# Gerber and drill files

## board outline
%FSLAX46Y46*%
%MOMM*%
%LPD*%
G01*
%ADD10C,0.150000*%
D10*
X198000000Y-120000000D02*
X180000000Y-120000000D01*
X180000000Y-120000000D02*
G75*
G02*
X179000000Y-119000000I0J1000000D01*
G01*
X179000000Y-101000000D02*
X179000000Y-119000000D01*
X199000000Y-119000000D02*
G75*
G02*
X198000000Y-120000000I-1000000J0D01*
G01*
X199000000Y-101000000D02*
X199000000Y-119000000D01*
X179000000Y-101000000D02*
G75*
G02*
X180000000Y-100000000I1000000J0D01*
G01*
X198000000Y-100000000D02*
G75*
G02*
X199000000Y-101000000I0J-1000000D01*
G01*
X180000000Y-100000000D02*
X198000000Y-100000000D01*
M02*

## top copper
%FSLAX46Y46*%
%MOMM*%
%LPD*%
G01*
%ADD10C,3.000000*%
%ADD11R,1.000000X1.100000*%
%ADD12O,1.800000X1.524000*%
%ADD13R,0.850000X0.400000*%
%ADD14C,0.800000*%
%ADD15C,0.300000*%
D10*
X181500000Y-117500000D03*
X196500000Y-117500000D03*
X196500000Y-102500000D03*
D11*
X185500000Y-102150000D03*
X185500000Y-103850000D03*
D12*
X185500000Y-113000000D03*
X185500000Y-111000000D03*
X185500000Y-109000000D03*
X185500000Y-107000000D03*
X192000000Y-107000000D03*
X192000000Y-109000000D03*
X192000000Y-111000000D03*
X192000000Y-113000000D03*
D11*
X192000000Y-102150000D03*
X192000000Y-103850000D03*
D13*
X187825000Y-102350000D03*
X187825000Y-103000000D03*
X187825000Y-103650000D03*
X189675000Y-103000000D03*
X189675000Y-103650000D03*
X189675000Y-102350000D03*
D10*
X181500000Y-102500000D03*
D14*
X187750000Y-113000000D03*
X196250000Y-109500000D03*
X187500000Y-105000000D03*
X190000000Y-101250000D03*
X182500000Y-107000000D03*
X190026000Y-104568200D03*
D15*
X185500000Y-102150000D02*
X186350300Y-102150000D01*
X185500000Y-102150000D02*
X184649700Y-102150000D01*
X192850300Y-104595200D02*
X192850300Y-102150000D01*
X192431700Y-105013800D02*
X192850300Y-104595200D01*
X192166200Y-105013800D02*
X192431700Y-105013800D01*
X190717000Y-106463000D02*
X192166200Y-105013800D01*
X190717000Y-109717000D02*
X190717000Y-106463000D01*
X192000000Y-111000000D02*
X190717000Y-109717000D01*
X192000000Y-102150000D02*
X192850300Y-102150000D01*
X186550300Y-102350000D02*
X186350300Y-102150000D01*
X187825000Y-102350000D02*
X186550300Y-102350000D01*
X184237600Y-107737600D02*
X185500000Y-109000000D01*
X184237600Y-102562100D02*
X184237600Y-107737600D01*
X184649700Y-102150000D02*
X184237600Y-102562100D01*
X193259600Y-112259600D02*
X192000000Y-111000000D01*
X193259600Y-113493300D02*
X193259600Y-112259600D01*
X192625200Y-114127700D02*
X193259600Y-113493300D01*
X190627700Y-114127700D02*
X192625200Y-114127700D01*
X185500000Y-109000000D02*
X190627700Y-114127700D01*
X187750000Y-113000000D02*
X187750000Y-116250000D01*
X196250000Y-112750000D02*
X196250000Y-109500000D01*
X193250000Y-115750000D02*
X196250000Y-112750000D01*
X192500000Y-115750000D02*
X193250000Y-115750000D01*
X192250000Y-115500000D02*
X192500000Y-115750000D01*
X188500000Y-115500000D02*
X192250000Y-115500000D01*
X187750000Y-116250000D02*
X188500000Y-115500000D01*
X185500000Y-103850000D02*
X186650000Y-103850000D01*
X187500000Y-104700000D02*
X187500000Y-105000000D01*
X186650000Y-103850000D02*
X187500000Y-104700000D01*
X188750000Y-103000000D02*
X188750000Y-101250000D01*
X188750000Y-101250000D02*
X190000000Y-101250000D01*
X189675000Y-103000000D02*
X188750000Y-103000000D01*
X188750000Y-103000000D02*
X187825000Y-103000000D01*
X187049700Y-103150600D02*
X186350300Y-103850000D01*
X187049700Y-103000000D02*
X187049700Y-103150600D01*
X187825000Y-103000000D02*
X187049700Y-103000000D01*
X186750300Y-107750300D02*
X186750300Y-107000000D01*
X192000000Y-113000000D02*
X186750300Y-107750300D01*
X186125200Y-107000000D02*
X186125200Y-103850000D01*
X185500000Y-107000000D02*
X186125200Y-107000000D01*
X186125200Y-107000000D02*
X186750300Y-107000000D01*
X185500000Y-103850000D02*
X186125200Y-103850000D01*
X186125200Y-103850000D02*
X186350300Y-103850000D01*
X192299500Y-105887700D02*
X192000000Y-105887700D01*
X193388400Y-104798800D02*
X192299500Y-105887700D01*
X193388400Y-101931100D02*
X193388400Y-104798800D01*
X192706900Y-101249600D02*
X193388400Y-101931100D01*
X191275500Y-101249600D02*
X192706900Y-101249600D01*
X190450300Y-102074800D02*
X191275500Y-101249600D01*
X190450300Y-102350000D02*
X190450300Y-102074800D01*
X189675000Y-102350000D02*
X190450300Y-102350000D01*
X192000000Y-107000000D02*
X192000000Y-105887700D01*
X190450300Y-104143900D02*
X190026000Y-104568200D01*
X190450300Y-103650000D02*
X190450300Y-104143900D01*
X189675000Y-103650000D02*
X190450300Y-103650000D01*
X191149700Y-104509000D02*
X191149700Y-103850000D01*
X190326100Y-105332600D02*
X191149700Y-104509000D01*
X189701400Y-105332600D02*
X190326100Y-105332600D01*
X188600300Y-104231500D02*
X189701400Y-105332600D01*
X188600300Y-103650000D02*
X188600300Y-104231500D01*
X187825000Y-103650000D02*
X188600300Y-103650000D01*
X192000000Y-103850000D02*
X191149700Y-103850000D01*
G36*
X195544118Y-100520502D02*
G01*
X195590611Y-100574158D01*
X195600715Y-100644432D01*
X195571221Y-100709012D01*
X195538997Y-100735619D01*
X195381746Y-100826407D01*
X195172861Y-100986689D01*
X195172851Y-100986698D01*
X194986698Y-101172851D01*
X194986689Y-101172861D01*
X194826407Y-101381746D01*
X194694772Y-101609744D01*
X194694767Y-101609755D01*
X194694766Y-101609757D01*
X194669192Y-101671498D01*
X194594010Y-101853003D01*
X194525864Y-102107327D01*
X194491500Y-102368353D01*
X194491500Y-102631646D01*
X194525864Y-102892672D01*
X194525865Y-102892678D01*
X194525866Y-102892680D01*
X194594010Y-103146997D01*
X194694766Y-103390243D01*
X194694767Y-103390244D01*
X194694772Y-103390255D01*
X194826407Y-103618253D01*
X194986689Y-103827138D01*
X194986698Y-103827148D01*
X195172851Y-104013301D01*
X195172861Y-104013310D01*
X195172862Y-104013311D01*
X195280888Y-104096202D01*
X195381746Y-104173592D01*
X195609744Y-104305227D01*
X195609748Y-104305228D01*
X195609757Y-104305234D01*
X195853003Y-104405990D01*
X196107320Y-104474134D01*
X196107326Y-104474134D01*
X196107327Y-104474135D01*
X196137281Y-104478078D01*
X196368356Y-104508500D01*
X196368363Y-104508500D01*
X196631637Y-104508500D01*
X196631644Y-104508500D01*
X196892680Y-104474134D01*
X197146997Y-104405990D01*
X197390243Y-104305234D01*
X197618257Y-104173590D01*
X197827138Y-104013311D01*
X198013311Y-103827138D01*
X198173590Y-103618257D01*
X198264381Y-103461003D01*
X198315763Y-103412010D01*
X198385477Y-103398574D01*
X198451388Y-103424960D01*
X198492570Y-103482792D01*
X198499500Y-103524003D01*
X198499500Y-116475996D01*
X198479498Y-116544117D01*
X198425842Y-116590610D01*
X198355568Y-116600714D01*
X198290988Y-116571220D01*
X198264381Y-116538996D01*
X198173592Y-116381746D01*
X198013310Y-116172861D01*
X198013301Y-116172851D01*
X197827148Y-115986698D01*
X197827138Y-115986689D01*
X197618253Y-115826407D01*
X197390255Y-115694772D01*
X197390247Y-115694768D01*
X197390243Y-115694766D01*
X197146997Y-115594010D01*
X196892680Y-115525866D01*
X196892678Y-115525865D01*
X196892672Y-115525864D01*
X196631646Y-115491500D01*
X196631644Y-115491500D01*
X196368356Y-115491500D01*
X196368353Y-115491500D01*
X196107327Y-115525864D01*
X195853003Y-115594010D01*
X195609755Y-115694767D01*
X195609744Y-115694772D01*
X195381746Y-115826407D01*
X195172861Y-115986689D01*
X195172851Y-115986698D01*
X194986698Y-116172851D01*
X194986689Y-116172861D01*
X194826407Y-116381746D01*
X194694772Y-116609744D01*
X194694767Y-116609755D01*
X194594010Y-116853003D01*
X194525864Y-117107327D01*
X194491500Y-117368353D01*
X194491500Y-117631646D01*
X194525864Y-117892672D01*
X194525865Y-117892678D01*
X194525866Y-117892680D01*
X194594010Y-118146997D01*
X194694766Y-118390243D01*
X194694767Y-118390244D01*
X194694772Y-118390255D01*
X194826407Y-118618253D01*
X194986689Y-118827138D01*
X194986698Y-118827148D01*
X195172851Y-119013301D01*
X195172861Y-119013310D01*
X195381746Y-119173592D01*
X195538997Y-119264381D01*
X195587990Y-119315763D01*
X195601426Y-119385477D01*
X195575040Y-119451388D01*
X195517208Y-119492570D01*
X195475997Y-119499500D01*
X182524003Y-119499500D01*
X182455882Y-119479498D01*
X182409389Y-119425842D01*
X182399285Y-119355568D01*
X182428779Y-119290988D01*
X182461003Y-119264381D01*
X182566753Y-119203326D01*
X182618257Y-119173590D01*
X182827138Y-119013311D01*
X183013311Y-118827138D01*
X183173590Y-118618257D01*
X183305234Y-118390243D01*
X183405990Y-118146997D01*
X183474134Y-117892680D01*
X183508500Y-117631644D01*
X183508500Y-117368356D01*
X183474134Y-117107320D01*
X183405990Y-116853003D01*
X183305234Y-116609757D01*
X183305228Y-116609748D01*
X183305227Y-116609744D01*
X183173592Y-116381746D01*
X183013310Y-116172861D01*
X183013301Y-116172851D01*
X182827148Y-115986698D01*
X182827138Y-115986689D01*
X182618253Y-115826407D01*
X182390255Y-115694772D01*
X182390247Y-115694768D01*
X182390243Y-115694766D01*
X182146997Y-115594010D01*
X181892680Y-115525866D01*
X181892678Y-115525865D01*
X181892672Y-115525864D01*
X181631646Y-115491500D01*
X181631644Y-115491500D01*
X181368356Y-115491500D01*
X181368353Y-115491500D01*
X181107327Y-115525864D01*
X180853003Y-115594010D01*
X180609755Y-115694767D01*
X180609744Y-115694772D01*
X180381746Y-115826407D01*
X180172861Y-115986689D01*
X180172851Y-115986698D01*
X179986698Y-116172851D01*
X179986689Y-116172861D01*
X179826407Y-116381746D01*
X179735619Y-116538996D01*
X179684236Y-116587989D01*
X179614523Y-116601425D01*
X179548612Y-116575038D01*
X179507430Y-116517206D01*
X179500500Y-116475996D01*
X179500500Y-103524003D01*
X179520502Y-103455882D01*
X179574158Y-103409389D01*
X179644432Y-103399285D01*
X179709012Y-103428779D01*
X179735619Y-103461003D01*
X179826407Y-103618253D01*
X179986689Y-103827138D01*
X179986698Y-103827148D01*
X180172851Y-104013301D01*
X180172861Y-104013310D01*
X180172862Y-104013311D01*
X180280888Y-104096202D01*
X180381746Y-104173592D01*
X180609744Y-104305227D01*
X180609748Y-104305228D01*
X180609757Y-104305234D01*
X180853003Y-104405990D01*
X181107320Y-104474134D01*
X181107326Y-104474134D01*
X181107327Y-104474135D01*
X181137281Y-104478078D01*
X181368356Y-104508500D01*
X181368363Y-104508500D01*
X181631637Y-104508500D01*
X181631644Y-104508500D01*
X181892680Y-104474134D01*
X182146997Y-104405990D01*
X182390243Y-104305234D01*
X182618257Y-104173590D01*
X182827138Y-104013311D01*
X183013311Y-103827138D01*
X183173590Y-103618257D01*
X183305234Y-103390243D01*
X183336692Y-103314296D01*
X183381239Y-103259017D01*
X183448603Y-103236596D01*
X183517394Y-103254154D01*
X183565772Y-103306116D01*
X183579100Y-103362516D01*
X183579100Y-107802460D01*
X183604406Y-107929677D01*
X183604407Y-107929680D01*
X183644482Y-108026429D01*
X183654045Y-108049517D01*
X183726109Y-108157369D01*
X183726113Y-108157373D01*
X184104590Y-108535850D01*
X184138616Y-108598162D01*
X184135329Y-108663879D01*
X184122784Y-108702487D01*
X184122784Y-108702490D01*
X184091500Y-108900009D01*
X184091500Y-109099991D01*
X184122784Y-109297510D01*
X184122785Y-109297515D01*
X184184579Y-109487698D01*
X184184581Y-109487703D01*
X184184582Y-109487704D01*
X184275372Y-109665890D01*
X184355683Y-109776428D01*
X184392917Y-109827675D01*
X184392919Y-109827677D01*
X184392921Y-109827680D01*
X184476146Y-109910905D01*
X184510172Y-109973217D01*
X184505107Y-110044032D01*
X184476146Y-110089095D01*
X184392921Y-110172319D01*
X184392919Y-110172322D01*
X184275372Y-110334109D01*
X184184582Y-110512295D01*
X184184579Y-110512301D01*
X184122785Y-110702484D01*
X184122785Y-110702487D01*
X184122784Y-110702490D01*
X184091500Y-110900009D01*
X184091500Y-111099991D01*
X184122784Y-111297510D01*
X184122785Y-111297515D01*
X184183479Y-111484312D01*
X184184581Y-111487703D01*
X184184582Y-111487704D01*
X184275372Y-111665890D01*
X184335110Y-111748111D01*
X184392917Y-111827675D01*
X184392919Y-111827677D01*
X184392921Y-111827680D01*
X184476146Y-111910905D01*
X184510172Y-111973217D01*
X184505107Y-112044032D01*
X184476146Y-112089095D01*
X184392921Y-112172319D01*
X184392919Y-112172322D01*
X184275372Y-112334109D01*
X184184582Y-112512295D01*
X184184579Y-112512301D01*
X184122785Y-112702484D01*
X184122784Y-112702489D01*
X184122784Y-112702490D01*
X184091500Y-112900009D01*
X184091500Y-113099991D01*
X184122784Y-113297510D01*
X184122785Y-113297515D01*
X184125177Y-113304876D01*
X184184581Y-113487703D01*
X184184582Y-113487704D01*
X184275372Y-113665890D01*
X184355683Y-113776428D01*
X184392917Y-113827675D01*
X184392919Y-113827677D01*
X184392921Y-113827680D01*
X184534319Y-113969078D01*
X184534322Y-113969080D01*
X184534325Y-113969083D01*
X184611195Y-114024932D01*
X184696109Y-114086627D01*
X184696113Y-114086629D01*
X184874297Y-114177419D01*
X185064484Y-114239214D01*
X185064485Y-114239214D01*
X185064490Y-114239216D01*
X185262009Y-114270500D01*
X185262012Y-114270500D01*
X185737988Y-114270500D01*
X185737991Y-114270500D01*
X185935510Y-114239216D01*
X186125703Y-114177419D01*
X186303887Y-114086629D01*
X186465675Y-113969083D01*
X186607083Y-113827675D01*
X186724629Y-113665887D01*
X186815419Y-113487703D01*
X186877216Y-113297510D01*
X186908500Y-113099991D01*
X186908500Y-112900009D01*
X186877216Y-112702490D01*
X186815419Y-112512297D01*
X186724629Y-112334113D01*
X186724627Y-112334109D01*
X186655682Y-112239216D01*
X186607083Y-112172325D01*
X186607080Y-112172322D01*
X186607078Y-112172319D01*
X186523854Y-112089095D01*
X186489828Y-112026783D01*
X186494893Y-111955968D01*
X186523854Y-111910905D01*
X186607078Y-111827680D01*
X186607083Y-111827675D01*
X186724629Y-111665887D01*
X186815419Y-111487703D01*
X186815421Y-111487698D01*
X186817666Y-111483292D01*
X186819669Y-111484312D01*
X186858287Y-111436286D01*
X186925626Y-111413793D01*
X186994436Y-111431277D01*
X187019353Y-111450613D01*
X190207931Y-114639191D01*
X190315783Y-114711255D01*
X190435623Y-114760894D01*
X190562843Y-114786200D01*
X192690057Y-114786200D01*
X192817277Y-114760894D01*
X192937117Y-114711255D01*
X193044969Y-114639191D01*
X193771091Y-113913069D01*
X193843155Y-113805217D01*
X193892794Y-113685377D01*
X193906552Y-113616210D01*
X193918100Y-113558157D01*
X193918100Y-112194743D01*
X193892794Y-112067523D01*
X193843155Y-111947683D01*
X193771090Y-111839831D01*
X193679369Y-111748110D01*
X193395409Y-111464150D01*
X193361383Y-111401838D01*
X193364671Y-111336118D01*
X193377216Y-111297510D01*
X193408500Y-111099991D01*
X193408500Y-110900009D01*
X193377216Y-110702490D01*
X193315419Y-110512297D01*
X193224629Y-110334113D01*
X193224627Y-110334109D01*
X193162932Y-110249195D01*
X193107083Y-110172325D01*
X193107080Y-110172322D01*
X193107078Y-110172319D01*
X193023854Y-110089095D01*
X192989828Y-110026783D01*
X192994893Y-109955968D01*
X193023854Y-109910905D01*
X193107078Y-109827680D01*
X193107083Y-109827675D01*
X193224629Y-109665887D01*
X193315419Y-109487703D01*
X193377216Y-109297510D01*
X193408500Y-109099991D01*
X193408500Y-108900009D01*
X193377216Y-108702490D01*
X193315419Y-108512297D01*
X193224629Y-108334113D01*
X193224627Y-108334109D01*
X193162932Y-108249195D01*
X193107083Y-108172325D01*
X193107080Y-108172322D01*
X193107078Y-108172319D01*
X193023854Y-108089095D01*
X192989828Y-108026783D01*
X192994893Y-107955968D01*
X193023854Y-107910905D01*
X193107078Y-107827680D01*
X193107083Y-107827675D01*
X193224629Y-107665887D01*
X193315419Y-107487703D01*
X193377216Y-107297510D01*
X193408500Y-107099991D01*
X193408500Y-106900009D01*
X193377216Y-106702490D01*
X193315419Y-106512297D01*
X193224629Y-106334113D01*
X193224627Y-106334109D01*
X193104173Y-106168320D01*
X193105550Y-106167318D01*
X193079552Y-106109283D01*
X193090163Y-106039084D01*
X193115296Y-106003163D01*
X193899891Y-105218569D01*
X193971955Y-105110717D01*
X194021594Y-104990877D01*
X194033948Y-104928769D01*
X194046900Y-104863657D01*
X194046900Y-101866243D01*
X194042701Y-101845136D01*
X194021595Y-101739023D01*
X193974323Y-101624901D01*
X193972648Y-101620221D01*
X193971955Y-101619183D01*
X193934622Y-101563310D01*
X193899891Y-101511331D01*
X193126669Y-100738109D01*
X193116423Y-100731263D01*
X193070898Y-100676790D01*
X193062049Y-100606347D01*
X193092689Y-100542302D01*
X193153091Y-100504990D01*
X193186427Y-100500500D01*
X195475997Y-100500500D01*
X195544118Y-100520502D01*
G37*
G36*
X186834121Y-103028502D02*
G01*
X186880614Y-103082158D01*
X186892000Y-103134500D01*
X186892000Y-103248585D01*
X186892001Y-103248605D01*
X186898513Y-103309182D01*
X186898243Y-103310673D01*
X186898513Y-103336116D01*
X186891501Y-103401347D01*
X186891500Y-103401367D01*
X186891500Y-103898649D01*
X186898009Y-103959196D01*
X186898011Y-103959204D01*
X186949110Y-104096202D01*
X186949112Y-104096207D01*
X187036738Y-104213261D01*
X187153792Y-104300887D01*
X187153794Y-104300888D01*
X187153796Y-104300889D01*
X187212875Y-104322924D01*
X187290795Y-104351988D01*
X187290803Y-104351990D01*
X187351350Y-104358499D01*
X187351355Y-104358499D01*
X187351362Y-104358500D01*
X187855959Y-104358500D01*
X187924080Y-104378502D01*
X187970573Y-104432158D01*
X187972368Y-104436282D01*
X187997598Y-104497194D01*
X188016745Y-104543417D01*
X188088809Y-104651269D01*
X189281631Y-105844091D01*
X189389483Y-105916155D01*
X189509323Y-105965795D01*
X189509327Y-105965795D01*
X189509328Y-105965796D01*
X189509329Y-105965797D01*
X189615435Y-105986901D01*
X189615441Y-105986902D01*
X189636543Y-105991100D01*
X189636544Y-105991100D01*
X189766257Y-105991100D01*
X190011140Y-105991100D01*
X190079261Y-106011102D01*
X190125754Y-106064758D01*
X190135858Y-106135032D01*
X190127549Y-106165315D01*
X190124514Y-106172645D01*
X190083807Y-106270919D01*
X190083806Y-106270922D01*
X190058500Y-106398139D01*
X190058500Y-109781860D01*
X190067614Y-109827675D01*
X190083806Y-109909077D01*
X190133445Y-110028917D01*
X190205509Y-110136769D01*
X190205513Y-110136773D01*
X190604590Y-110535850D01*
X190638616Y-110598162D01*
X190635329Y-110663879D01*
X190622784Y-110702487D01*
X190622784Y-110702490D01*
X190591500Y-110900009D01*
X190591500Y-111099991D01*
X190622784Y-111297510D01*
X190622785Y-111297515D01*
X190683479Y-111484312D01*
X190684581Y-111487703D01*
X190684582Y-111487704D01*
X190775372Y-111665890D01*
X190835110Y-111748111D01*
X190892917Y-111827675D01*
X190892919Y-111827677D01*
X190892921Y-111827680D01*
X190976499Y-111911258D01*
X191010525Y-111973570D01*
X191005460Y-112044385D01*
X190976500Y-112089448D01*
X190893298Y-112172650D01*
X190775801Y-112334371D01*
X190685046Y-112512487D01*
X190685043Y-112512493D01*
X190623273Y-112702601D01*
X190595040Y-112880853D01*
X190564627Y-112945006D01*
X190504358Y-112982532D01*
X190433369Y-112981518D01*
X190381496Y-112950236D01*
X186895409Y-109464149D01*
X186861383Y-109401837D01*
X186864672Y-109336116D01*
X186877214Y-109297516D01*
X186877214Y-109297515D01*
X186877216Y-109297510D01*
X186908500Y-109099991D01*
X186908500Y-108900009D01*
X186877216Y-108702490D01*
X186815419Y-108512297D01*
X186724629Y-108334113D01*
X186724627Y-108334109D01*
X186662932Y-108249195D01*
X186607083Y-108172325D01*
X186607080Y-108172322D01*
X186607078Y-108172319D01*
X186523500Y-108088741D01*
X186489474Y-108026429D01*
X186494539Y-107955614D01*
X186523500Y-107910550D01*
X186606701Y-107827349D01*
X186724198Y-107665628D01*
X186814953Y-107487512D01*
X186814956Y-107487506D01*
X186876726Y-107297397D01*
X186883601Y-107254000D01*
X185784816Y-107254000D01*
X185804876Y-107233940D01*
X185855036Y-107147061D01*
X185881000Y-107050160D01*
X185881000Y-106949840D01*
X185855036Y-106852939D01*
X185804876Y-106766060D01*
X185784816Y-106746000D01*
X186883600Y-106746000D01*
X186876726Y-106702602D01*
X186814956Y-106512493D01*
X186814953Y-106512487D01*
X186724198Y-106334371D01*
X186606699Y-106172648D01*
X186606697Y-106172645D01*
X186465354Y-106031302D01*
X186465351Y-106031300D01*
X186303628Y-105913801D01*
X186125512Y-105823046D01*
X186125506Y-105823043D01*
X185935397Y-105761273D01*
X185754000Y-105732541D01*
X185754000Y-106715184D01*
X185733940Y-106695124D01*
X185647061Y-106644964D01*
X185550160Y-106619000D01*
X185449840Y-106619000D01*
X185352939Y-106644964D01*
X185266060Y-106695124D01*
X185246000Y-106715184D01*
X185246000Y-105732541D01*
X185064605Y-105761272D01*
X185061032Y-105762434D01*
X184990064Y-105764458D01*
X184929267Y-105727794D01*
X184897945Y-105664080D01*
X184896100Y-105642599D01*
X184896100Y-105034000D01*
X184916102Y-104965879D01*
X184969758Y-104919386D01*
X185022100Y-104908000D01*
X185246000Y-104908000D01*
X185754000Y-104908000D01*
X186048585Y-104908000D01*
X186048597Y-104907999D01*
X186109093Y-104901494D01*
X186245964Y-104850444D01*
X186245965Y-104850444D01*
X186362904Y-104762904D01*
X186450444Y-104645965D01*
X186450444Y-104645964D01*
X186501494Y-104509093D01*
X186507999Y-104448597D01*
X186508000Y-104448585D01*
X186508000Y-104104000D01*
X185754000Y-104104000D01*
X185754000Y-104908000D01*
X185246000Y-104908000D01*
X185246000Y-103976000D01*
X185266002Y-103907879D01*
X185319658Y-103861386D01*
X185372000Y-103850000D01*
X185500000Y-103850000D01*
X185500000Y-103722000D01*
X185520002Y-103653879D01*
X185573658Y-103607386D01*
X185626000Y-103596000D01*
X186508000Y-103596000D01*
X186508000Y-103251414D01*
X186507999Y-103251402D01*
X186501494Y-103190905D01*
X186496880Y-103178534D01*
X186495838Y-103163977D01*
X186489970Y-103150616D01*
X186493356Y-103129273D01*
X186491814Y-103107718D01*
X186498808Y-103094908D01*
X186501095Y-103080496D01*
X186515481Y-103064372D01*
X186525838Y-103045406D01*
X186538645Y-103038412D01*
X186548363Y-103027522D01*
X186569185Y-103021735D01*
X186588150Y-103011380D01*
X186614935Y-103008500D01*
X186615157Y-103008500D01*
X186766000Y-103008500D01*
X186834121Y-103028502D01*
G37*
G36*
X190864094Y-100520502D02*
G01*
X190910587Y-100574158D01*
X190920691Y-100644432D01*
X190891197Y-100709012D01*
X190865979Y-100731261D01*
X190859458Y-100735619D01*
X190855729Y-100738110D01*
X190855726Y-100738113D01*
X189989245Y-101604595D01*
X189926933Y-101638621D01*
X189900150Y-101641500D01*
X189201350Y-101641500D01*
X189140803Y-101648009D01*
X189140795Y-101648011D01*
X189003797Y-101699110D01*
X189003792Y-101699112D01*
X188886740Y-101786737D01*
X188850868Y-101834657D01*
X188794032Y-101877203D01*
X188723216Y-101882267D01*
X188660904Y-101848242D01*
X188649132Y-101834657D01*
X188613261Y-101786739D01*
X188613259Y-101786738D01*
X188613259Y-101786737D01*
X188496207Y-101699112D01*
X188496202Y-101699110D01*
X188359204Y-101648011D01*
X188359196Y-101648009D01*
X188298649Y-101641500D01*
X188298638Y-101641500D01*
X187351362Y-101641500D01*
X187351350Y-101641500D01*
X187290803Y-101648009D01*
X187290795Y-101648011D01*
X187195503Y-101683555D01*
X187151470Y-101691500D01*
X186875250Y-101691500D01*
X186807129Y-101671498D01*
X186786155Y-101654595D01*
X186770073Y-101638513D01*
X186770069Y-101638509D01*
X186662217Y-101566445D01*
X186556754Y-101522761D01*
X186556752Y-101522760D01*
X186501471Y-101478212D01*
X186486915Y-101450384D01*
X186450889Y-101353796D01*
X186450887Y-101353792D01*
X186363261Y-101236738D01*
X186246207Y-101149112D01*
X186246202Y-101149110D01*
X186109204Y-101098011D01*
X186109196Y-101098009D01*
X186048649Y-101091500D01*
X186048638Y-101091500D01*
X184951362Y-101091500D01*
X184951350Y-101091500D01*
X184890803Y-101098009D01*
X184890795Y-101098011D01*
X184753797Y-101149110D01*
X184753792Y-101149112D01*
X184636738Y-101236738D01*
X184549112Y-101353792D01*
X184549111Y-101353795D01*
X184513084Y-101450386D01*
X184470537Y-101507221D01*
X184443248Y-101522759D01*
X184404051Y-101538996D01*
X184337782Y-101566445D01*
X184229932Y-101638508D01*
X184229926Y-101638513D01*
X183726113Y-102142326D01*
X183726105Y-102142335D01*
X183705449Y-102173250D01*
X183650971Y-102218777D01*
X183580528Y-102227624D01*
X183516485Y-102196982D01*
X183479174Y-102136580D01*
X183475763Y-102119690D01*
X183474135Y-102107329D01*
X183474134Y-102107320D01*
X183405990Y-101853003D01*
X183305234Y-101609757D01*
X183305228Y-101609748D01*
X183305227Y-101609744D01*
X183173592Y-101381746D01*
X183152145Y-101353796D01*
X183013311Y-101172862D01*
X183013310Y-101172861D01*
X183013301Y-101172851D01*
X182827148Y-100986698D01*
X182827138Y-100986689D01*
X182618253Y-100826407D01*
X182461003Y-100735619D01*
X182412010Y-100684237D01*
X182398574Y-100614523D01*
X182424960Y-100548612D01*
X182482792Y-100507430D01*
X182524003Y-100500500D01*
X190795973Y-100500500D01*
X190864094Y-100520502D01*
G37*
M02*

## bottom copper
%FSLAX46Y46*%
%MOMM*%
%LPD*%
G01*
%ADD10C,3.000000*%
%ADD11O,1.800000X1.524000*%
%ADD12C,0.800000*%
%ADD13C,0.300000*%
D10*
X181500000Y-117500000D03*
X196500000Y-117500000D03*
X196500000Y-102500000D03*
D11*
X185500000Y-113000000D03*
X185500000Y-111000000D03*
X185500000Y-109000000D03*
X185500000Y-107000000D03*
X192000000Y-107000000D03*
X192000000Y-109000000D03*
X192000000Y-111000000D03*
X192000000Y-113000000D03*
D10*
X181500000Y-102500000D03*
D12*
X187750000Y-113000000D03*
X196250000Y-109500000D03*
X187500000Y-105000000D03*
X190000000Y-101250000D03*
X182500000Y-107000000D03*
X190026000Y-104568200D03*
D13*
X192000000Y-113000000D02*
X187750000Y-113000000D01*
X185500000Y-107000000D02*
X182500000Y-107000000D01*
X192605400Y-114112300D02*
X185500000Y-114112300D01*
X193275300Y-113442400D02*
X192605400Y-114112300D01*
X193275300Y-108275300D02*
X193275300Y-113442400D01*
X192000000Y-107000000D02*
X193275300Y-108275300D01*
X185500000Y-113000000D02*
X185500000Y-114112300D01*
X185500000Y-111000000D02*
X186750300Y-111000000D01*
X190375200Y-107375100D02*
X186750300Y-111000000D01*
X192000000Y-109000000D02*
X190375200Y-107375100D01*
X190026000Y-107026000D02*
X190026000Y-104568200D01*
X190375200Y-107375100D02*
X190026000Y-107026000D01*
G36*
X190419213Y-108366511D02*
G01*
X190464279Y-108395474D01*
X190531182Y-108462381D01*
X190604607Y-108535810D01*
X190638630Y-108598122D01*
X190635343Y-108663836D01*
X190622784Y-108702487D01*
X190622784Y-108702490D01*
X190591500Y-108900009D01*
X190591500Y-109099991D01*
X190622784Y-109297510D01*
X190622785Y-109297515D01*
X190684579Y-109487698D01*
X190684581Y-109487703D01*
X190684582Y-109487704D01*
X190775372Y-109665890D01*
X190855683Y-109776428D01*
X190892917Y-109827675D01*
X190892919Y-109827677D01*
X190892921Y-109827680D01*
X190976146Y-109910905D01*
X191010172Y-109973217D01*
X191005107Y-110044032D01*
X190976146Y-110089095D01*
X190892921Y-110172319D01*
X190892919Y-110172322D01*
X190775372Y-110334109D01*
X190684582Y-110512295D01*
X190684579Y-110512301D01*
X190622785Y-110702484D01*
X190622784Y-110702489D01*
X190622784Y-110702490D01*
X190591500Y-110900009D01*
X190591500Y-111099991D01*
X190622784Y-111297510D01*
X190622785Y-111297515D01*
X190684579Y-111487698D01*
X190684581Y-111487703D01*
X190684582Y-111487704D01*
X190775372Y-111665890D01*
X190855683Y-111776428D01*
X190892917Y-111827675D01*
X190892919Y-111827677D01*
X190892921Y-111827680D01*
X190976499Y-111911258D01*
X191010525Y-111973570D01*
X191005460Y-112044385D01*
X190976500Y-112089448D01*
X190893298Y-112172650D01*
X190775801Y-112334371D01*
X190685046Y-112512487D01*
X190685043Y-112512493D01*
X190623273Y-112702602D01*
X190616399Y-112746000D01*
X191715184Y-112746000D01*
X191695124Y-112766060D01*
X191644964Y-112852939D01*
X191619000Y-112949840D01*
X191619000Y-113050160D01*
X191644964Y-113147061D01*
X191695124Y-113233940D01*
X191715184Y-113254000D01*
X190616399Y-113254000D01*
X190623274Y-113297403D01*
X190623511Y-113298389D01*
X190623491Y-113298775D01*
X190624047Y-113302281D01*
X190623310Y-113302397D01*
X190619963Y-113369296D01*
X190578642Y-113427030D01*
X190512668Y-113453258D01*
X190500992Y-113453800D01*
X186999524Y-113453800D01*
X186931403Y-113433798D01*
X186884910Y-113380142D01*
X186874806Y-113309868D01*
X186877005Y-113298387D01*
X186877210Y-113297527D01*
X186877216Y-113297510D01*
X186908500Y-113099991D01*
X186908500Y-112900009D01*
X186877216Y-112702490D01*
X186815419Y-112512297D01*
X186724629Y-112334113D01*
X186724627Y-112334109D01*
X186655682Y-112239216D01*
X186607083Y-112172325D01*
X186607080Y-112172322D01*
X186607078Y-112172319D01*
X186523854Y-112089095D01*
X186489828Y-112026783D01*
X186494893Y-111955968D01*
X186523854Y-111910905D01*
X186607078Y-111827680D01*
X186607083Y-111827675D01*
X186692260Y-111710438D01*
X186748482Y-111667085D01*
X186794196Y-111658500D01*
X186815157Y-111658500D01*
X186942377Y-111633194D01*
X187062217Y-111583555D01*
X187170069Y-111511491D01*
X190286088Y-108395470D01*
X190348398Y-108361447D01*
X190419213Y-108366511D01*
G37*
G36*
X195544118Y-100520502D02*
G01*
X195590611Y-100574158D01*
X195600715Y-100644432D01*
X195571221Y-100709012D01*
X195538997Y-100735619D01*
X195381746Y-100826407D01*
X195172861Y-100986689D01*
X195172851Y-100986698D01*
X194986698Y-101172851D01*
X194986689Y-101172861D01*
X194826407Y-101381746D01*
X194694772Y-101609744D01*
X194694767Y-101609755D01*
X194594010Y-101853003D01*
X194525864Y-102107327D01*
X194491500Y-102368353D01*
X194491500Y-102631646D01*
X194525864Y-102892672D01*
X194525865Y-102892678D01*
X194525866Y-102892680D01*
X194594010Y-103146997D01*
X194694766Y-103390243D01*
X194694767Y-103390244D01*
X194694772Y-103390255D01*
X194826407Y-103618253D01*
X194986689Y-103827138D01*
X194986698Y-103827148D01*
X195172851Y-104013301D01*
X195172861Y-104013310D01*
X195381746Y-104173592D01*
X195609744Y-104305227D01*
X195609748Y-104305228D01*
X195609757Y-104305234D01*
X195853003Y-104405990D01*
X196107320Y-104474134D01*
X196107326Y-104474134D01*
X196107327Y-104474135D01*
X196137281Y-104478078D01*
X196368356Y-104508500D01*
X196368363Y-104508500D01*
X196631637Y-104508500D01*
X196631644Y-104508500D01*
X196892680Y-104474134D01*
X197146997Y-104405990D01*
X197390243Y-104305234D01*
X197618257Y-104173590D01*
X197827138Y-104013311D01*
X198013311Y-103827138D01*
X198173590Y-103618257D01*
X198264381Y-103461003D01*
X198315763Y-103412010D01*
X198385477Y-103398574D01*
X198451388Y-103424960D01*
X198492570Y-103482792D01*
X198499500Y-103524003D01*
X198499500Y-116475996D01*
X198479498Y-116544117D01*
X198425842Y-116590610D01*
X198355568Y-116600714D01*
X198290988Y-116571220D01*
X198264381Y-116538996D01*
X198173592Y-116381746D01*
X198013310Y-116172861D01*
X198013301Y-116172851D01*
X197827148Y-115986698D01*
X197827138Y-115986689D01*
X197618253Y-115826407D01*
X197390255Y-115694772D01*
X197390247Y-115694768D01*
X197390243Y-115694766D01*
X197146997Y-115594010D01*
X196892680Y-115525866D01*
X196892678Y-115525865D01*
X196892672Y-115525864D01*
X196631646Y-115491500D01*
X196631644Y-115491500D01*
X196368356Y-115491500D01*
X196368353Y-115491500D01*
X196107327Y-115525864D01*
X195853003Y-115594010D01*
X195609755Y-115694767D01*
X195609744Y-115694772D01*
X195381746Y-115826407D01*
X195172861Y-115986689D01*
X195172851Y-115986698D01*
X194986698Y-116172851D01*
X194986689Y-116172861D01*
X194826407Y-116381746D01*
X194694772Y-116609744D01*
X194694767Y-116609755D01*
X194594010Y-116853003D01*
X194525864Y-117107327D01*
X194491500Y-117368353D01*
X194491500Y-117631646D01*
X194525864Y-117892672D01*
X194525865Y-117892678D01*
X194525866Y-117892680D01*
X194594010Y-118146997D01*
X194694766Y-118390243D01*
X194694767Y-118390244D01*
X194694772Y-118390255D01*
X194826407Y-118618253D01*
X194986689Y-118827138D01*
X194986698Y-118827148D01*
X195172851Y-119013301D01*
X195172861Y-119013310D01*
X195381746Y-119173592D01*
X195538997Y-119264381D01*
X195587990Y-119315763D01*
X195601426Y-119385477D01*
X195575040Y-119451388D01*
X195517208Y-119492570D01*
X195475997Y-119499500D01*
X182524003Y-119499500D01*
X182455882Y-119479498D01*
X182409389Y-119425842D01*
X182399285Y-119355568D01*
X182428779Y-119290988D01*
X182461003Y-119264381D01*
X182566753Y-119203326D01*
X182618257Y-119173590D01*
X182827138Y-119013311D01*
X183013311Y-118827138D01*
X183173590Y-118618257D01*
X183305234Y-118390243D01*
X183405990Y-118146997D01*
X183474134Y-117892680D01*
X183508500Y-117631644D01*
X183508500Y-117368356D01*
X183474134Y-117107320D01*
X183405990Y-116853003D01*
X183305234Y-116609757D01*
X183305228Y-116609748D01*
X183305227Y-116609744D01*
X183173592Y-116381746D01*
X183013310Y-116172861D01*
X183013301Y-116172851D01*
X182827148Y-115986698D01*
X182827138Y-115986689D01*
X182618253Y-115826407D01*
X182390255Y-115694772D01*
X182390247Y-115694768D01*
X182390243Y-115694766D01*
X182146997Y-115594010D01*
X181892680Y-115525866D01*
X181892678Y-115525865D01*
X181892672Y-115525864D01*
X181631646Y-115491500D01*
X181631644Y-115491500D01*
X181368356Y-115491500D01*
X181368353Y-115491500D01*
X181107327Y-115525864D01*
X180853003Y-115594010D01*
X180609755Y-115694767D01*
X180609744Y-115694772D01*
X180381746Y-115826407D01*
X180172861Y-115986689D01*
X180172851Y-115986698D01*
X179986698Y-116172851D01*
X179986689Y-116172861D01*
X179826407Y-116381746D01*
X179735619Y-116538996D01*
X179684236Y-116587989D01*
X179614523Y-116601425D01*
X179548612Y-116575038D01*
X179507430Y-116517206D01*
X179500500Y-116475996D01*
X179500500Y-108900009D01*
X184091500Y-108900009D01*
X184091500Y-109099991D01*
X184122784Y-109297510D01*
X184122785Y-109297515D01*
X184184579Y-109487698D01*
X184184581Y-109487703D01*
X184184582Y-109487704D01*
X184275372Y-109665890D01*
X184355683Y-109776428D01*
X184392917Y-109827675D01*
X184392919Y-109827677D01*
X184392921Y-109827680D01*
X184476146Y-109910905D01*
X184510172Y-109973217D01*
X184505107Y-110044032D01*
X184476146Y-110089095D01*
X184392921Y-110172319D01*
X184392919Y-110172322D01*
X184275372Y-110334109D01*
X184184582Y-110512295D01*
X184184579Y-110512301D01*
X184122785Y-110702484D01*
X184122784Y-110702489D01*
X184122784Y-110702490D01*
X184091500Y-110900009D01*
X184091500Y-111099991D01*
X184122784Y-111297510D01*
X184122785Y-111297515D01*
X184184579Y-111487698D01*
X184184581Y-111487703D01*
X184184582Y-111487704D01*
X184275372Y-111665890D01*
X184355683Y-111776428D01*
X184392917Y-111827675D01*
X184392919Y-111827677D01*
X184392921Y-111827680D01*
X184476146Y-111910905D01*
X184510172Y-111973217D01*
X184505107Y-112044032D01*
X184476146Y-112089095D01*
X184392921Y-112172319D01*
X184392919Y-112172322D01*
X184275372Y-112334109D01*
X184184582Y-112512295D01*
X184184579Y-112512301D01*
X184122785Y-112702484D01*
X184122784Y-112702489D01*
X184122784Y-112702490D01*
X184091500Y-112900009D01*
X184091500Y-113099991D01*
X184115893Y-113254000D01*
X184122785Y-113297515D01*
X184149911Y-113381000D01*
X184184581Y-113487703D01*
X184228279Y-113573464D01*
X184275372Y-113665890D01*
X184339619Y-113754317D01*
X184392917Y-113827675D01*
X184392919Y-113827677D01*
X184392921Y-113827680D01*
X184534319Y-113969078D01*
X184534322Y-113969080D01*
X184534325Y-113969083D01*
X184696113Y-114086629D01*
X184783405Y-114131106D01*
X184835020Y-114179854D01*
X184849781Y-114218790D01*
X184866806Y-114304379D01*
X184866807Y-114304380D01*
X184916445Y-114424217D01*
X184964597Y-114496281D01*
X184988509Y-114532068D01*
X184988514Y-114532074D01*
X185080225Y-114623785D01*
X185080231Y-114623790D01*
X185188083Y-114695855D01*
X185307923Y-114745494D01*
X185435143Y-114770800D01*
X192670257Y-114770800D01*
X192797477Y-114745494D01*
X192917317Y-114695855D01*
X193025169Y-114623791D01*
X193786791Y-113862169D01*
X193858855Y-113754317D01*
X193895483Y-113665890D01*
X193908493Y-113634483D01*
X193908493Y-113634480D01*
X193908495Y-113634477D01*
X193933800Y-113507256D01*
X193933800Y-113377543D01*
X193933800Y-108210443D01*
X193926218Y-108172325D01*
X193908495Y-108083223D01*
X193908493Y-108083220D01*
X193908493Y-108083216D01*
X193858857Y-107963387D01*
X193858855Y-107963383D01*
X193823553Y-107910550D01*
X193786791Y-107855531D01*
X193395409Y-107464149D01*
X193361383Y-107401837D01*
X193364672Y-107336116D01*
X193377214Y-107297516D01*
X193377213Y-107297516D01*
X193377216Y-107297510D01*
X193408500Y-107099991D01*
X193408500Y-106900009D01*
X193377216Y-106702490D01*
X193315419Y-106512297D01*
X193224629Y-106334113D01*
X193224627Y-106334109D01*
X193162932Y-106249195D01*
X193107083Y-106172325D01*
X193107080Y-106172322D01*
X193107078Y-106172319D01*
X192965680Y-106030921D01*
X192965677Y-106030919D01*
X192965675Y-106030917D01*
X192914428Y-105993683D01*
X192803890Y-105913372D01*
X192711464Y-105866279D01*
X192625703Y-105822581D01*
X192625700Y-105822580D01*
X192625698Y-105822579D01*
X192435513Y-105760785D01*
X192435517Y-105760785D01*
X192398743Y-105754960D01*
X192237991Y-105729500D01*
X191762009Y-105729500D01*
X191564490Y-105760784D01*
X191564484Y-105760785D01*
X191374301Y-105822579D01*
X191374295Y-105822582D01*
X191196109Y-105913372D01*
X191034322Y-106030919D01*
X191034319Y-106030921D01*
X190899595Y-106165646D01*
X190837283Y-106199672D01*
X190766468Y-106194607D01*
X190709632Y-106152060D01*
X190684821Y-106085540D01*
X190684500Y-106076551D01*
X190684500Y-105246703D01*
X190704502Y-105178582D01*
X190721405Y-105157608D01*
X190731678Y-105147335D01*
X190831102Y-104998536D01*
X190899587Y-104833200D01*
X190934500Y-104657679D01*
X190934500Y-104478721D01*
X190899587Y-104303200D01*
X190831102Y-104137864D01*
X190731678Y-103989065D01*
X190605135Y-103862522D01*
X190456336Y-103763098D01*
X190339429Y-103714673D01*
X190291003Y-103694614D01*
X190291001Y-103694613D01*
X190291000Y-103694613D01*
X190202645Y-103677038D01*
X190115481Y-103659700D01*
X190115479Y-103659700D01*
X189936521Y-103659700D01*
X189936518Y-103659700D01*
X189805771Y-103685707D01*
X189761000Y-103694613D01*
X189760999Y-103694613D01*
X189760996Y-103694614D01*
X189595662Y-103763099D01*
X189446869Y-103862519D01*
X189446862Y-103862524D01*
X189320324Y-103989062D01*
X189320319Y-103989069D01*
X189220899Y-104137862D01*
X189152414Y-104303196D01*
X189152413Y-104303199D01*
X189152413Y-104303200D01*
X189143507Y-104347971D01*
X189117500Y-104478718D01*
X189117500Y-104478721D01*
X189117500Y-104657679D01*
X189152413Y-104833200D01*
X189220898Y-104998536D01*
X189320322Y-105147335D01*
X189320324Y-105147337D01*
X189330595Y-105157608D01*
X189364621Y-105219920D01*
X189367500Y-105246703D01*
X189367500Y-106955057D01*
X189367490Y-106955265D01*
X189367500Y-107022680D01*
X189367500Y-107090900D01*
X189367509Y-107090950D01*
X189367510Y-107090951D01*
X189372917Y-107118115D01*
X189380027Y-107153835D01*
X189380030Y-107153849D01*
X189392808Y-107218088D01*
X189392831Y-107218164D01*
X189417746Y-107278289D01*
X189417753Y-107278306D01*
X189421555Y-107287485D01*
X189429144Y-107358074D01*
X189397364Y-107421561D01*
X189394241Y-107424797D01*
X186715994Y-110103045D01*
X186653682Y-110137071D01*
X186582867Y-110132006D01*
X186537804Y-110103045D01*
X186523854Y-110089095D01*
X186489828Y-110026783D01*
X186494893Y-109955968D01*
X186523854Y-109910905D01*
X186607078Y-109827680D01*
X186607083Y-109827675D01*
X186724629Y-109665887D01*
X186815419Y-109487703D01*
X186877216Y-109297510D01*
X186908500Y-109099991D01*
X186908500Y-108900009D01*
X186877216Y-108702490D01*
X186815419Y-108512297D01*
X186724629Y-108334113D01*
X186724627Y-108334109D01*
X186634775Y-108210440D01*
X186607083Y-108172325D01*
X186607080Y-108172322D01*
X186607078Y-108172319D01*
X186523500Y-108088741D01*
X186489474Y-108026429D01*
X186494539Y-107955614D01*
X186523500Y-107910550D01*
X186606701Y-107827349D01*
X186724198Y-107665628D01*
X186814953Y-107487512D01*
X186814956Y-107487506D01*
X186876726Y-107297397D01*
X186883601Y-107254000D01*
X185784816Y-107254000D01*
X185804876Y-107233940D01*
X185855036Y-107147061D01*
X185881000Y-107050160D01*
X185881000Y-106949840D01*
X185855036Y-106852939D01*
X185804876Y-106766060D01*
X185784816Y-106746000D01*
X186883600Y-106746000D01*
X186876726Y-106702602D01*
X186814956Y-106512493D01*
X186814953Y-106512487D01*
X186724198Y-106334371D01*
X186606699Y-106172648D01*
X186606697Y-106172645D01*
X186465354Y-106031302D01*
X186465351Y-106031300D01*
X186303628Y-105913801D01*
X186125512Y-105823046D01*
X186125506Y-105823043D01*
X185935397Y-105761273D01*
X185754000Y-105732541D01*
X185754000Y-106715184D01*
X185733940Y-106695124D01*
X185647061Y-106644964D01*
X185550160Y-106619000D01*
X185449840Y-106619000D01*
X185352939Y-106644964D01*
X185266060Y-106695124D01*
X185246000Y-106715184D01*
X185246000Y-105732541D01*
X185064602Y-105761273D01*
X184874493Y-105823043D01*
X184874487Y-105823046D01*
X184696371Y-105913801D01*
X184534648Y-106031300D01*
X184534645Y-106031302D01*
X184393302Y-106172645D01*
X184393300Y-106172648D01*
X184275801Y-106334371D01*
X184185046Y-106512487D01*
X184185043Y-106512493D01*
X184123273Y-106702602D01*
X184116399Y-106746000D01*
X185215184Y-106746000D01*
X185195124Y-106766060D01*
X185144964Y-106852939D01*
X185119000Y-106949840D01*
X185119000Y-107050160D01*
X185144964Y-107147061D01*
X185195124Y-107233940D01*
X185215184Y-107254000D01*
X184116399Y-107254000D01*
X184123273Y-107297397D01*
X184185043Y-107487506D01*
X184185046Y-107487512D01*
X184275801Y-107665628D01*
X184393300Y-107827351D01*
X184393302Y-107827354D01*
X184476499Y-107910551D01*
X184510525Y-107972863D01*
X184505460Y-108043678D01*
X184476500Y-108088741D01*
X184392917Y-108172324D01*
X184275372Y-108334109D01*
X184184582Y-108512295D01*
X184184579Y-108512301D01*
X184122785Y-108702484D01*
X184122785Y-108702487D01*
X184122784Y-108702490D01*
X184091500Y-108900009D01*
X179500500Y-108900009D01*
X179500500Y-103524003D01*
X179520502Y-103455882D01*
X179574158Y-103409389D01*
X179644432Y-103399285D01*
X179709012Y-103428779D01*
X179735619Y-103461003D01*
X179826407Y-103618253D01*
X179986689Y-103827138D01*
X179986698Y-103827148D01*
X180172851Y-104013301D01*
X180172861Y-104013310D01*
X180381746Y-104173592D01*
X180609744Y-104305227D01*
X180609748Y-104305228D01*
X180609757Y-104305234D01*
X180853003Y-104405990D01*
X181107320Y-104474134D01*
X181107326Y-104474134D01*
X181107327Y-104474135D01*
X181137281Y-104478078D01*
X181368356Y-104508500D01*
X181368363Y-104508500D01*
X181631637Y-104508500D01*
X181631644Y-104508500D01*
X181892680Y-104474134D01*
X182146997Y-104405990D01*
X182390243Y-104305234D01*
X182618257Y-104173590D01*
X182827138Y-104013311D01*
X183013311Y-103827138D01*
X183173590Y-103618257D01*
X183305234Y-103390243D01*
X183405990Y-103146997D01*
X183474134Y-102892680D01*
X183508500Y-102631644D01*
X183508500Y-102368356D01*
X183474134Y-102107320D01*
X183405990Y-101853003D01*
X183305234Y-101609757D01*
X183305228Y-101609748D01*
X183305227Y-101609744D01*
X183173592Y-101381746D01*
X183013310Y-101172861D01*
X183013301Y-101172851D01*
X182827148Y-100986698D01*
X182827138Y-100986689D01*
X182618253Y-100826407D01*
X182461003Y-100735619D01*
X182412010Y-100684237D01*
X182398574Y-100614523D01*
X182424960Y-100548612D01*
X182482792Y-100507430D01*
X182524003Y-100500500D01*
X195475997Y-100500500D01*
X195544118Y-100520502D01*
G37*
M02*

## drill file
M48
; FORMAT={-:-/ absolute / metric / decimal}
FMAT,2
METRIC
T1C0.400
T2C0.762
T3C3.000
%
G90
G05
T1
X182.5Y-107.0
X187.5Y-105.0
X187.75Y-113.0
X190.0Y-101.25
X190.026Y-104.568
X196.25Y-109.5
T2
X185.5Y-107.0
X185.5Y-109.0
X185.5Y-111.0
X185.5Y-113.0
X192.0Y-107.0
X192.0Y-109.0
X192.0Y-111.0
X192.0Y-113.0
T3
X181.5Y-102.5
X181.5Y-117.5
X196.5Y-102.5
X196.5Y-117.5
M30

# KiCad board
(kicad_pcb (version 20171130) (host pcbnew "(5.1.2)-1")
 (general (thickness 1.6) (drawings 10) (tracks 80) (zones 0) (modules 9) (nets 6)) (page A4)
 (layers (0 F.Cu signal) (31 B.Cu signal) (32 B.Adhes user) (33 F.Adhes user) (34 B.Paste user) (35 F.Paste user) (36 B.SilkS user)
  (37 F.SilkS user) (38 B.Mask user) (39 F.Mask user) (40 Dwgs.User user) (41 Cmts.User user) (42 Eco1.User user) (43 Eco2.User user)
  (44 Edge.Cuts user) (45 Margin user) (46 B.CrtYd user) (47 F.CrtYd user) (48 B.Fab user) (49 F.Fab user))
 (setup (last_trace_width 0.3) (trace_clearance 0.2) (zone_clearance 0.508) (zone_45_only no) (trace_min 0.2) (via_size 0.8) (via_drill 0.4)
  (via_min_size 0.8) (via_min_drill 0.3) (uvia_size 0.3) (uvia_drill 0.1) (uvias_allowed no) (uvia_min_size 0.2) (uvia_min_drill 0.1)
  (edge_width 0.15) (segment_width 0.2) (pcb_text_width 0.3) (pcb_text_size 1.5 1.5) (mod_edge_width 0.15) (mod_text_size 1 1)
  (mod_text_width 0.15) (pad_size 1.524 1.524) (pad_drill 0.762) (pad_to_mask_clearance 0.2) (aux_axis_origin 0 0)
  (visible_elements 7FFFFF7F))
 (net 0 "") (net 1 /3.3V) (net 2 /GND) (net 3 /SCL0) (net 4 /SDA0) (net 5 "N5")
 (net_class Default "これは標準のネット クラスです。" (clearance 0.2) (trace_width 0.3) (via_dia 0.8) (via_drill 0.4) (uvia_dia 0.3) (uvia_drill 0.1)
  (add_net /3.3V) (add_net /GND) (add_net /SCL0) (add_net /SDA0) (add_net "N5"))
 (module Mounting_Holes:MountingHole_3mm (layer F.Cu) (at 181.5 117.5)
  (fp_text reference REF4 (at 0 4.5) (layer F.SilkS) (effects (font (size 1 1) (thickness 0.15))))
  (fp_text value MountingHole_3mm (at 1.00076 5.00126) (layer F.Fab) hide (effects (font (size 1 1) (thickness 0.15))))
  (pad 1 thru_hole circle (at 0 0) (size 3 3) (drill 3) (layers)))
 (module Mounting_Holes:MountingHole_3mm (layer F.Cu) (at 196.5 117.5)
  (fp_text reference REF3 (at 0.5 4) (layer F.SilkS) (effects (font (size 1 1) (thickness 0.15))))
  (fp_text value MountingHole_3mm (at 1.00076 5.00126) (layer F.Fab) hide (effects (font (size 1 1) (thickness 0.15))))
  (pad 1 thru_hole circle (at 0 0) (size 3 3) (drill 3) (layers)))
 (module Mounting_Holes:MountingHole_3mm (layer F.Cu) (at 196.5 102.5)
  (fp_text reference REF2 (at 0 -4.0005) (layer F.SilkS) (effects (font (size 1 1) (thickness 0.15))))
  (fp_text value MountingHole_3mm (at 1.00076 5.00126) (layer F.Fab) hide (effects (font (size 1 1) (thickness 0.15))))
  (pad 1 thru_hole circle (at 0 0) (size 3 3) (drill 3) (layers)))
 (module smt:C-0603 (layer F.Cu) (at 185.5 103 270)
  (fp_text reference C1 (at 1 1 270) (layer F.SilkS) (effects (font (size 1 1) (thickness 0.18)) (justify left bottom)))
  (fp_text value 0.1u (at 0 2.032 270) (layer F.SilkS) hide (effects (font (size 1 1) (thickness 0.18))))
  (pad 1 smd rect (at -0.85 0 270) (size 1.1 1) (layers F.Cu F.Paste F.Mask) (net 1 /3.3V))
  (pad 2 smd rect (at 0.85 0 270) (size 1.1 1) (layers F.Cu F.Paste F.Mask) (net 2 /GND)))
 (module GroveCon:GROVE (layer F.Cu) (at 185.5 113 90)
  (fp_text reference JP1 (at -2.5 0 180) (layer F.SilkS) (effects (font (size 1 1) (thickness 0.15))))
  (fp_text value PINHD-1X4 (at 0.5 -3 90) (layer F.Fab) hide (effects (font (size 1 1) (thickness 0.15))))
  (pad 1 thru_hole oval (at 0 0 90) (size 1.524 1.8) (drill 0.762) (layers *.Cu *.Paste *.Mask F.SilkS) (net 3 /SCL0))
  (pad 2 thru_hole oval (at 2 0 90) (size 1.524 1.8) (drill 0.762) (layers *.Cu *.Paste *.Mask F.SilkS) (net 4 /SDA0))
  (pad 3 thru_hole oval (at 4 0 90) (size 1.524 1.8) (drill 0.762) (layers *.Cu *.Paste *.Mask F.SilkS) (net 1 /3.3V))
  (pad 4 thru_hole oval (at 6 0 90) (size 1.524 1.8) (drill 0.762) (layers *.Cu *.Paste *.Mask F.SilkS) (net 2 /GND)))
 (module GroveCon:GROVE (layer F.Cu) (at 192 107 270)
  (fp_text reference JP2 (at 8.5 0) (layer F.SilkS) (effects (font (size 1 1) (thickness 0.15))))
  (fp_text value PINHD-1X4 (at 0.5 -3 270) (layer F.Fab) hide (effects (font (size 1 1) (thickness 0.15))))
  (pad 1 thru_hole oval (at 0 0 270) (size 1.524 1.8) (drill 0.762) (layers *.Cu *.Paste *.Mask F.SilkS) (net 3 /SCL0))
  (pad 2 thru_hole oval (at 2 0 270) (size 1.524 1.8) (drill 0.762) (layers *.Cu *.Paste *.Mask F.SilkS) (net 4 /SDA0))
  (pad 3 thru_hole oval (at 4 0 270) (size 1.524 1.8) (drill 0.762) (layers *.Cu *.Paste *.Mask F.SilkS) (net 1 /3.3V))
  (pad 4 thru_hole oval (at 6 0 270) (size 1.524 1.8) (drill 0.762) (layers *.Cu *.Paste *.Mask F.SilkS) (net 2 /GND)))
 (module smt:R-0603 (layer F.Cu) (at 192 103 270)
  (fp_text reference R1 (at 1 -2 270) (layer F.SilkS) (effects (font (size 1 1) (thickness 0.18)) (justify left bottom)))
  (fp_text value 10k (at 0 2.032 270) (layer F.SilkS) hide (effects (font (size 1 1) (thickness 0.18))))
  (pad 1 smd rect (at -0.85 0 270) (size 1.1 1) (layers F.Cu F.Paste F.Mask) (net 1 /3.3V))
  (pad 2 smd rect (at 0.85 0 270) (size 1.1 1) (layers F.Cu F.Paste F.Mask) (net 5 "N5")))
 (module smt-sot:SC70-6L (layer F.Cu) (at 188.75 103 270)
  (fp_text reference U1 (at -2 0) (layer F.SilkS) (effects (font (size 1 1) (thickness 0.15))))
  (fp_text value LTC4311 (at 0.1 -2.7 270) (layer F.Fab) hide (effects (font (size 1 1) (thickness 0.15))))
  (pad 1 smd rect (at -0.65 0.925 270) (size 0.4 0.85) (layers F.Cu F.Paste F.Mask) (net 1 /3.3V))
  (pad 2 smd rect (at 0 0.925 270) (size 0.4 0.85) (layers F.Cu F.Paste F.Mask) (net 2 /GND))
  (pad 3 smd rect (at 0.65 0.925 270) (size 0.4 0.85) (layers F.Cu F.Paste F.Mask) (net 5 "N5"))
  (pad 5 smd rect (at 0 -0.925 270) (size 0.4 0.85) (layers F.Cu F.Paste F.Mask) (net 2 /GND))
  (pad 4 smd rect (at 0.65 -0.925 270) (size 0.4 0.85) (layers F.Cu F.Paste F.Mask) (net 4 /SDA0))
  (pad 6 smd rect (at -0.65 -0.925 270) (size 0.4 0.85) (layers F.Cu F.Paste F.Mask) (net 3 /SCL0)))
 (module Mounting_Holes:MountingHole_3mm (layer F.Cu) (at 181.5 102.5)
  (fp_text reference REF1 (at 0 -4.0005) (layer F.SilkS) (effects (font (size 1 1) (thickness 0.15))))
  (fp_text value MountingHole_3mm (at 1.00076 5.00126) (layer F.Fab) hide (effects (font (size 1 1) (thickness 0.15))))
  (pad 1 thru_hole circle (at 0 0) (size 3 3) (drill 3) (layers)))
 (gr_line (start 198 120) (end 180 120) (angle 90) (layer Edge.Cuts) (width 0.15))
 (gr_arc (start 180 119) (end 180 120) (angle 90) (layer Edge.Cuts) (width 0.15))
 (gr_line (start 179 101) (end 179 119) (angle 90) (layer Edge.Cuts) (width 0.15))
 (gr_arc (start 198 119) (end 199 119) (angle 90) (layer Edge.Cuts) (width 0.15))
 (gr_line (start 199 101) (end 199 119) (angle 90) (layer Edge.Cuts) (width 0.15))
 (gr_arc (start 180 101) (end 179 101) (angle 90) (layer Edge.Cuts) (width 0.15))
 (gr_arc (start 198 101) (end 198 100) (angle 90) (layer Edge.Cuts) (width 0.15))
 (gr_line (start 180 100) (end 198 100) (angle 90) (layer Edge.Cuts) (width 0.15))
 (segment (start 185.5 102.15) (end 186.3503 102.15) (width 0.3) (layer F.Cu) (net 1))
 (segment (start 185.5 102.15) (end 184.6497 102.15) (width 0.3) (layer F.Cu) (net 1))
 (segment (start 192.8503 104.5952) (end 192.8503 102.15) (width 0.3) (layer F.Cu) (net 1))
 (segment (start 192.4317 105.0138) (end 192.8503 104.5952) (width 0.3) (layer F.Cu) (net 1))
 (segment (start 192.1662 105.0138) (end 192.4317 105.0138) (width 0.3) (layer F.Cu) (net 1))
 (segment (start 190.717 106.463) (end 192.1662 105.0138) (width 0.3) (layer F.Cu) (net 1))
 (segment (start 190.717 109.717) (end 190.717 106.463) (width 0.3) (layer F.Cu) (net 1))
 (segment (start 192 111) (end 190.717 109.717) (width 0.3) (layer F.Cu) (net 1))
 (segment (start 192 102.15) (end 192.8503 102.15) (width 0.3) (layer F.Cu) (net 1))
 (segment (start 186.5503 102.35) (end 186.3503 102.15) (width 0.3) (layer F.Cu) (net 1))
 (segment (start 187.825 102.35) (end 186.5503 102.35) (width 0.3) (layer F.Cu) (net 1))
 (segment (start 184.2376 107.7376) (end 185.5 109) (width 0.3) (layer F.Cu) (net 1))
 (segment (start 184.2376 102.5621) (end 184.2376 107.7376) (width 0.3) (layer F.Cu) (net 1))
 (segment (start 184.6497 102.15) (end 184.2376 102.5621) (width 0.3) (layer F.Cu) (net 1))
 (segment (start 193.2596 112.2596) (end 192 111) (width 0.3) (layer F.Cu) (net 1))
 (segment (start 193.2596 113.4933) (end 193.2596 112.2596) (width 0.3) (layer F.Cu) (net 1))
 (segment (start 192.6252 114.1277) (end 193.2596 113.4933) (width 0.3) (layer F.Cu) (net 1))
 (segment (start 190.6277 114.1277) (end 192.6252 114.1277) (width 0.3) (layer F.Cu) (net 1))
 (segment (start 185.5 109) (end 190.6277 114.1277) (width 0.3) (layer F.Cu) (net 1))
 (segment (start 187.75 113) (end 187.75 116.25) (width 0.3) (layer F.Cu) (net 2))
 (via (at 187.75 113) (size 0.8) (drill 0.4) (layers F.Cu B.Cu) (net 2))
 (segment (start 192 113) (end 187.75 113) (width 0.3) (layer B.Cu) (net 2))
 (via (at 196.25 109.5) (size 0.8) (drill 0.4) (layers F.Cu B.Cu) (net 2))
 (segment (start 196.25 112.75) (end 196.25 109.5) (width 0.3) (layer F.Cu) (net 2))
 (segment (start 193.25 115.75) (end 196.25 112.75) (width 0.3) (layer F.Cu) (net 2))
 (segment (start 192.5 115.75) (end 193.25 115.75) (width 0.3) (layer F.Cu) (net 2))
 (segment (start 192.25 115.5) (end 192.5 115.75) (width 0.3) (layer F.Cu) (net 2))
 (segment (start 188.5 115.5) (end 192.25 115.5) (width 0.3) (layer F.Cu) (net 2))
 (segment (start 187.75 116.25) (end 188.5 115.5) (width 0.3) (layer F.Cu) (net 2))
 (segment (start 185.5 103.85) (end 186.65 103.85) (width 0.3) (layer F.Cu) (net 2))
 (via (at 187.5 105) (size 0.8) (drill 0.4) (layers F.Cu B.Cu) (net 2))
 (segment (start 187.5 104.7) (end 187.5 105) (width 0.3) (layer F.Cu) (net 2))
 (segment (start 186.65 103.85) (end 187.5 104.7) (width 0.3) (layer F.Cu) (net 2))
 (segment (start 188.75 103) (end 188.75 101.25) (width 0.3) (layer F.Cu) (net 2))
 (via (at 190 101.25) (size 0.8) (drill 0.4) (layers F.Cu B.Cu) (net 2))
 (segment (start 188.75 101.25) (end 190 101.25) (width 0.3) (layer F.Cu) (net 2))
 (segment (start 185.5 107) (end 182.5 107) (width 0.3) (layer B.Cu) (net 2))
 (via (at 182.5 107) (size 0.8) (drill 0.4) (layers F.Cu B.Cu) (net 2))
 (segment (start 189.675 103) (end 188.75 103) (width 0.3) (layer F.Cu) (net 2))
 (segment (start 188.75 103) (end 187.825 103) (width 0.3) (layer F.Cu) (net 2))
 (segment (start 187.0497 103.1506) (end 186.3503 103.85) (width 0.3) (layer F.Cu) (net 2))
 (segment (start 187.0497 103) (end 187.0497 103.1506) (width 0.3) (layer F.Cu) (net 2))
 (segment (start 187.825 103) (end 187.0497 103) (width 0.3) (layer F.Cu) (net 2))
 (segment (start 186.7503 107.7503) (end 186.7503 107) (width 0.3) (layer F.Cu) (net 2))
 (segment (start 192 113) (end 186.7503 107.7503) (width 0.3) (layer F.Cu) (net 2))
 (segment (start 186.1252 107) (end 186.1252 103.85) (width 0.3) (layer F.Cu) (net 2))
 (segment (start 185.5 107) (end 186.1252 107) (width 0.3) (layer F.Cu) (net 2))
 (segment (start 186.1252 107) (end 186.7503 107) (width 0.3) (layer F.Cu) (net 2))
 (segment (start 185.5 103.85) (end 186.1252 103.85) (width 0.3) (layer F.Cu) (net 2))
 (segment (start 186.1252 103.85) (end 186.3503 103.85) (width 0.3) (layer F.Cu) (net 2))
 (segment (start 192.6054 114.1123) (end 185.5 114.1123) (width 0.3) (layer B.Cu) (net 3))
 (segment (start 193.2753 113.4424) (end 192.6054 114.1123) (width 0.3) (layer B.Cu) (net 3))
 (segment (start 193.2753 108.2753) (end 193.2753 113.4424) (width 0.3) (layer B.Cu) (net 3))
 (segment (start 192 107) (end 193.2753 108.2753) (width 0.3) (layer B.Cu) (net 3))
 (segment (start 185.5 113) (end 185.5 114.1123) (width 0.3) (layer B.Cu) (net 3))
 (segment (start 192.2995 105.8877) (end 192 105.8877) (width 0.3) (layer F.Cu) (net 3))
 (segment (start 193.3884 104.7988) (end 192.2995 105.8877) (width 0.3) (layer F.Cu) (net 3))
 (segment (start 193.3884 101.9311) (end 193.3884 104.7988) (width 0.3) (layer F.Cu) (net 3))
 (segment (start 192.7069 101.2496) (end 193.3884 101.9311) (width 0.3) (layer F.Cu) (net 3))
 (segment (start 191.2755 101.2496) (end 192.7069 101.2496) (width 0.3) (layer F.Cu) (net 3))
 (segment (start 190.4503 102.0748) (end 191.2755 101.2496) (width 0.3) (layer F.Cu) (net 3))
 (segment (start 190.4503 102.35) (end 190.4503 102.0748) (width 0.3) (layer F.Cu) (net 3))
 (segment (start 189.675 102.35) (end 190.4503 102.35) (width 0.3) (layer F.Cu) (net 3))
 (segment (start 192 107) (end 192 105.8877) (width 0.3) (layer F.Cu) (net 3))
 (via (at 190.026 104.5682) (size 0.8) (layers F.Cu B.Cu) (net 4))
 (segment (start 190.4503 104.1439) (end 190.026 104.5682) (width 0.3) (layer F.Cu) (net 4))
 (segment (start 190.4503 103.65) (end 190.4503 104.1439) (width 0.3) (layer F.Cu) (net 4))
 (segment (start 189.675 103.65) (end 190.4503 103.65) (width 0.3) (layer F.Cu) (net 4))
 (segment (start 185.5 111) (end 186.7503 111) (width 0.3) (layer B.Cu) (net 4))
 (segment (start 190.3752 107.3751) (end 186.7503 111) (width 0.3) (layer B.Cu) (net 4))
 (segment (start 192 109) (end 190.3752 107.3751) (width 0.3) (layer B.Cu) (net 4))
 (segment (start 190.026 107.026) (end 190.026 104.5682) (width 0.3) (layer B.Cu) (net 4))
 (segment (start 190.3752 107.3751) (end 190.026 107.026) (width 0.3) (layer B.Cu) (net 4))
 (segment (start 191.1497 104.509) (end 191.1497 103.85) (width 0.3) (layer F.Cu) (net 5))
 (segment (start 190.3261 105.3326) (end 191.1497 104.509) (width 0.3) (layer F.Cu) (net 5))
 (segment (start 189.7014 105.3326) (end 190.3261 105.3326) (width 0.3) (layer F.Cu) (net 5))
 (segment (start 188.6003 104.2315) (end 189.7014 105.3326) (width 0.3) (layer F.Cu) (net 5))
 (segment (start 188.6003 103.65) (end 188.6003 104.2315) (width 0.3) (layer F.Cu) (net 5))
 (segment (start 187.825 103.65) (end 188.6003 103.65) (width 0.3) (layer F.Cu) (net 5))
 (segment (start 192 103.85) (end 191.1497 103.85) (width 0.3) (layer F.Cu) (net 5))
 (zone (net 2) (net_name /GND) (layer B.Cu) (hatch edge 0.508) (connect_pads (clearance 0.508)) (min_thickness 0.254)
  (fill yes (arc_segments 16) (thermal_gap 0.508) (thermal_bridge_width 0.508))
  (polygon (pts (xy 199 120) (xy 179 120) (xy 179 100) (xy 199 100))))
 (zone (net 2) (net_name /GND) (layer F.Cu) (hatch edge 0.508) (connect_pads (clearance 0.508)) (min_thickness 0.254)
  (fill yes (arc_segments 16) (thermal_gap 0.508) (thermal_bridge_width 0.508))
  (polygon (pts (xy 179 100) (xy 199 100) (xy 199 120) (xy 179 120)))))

